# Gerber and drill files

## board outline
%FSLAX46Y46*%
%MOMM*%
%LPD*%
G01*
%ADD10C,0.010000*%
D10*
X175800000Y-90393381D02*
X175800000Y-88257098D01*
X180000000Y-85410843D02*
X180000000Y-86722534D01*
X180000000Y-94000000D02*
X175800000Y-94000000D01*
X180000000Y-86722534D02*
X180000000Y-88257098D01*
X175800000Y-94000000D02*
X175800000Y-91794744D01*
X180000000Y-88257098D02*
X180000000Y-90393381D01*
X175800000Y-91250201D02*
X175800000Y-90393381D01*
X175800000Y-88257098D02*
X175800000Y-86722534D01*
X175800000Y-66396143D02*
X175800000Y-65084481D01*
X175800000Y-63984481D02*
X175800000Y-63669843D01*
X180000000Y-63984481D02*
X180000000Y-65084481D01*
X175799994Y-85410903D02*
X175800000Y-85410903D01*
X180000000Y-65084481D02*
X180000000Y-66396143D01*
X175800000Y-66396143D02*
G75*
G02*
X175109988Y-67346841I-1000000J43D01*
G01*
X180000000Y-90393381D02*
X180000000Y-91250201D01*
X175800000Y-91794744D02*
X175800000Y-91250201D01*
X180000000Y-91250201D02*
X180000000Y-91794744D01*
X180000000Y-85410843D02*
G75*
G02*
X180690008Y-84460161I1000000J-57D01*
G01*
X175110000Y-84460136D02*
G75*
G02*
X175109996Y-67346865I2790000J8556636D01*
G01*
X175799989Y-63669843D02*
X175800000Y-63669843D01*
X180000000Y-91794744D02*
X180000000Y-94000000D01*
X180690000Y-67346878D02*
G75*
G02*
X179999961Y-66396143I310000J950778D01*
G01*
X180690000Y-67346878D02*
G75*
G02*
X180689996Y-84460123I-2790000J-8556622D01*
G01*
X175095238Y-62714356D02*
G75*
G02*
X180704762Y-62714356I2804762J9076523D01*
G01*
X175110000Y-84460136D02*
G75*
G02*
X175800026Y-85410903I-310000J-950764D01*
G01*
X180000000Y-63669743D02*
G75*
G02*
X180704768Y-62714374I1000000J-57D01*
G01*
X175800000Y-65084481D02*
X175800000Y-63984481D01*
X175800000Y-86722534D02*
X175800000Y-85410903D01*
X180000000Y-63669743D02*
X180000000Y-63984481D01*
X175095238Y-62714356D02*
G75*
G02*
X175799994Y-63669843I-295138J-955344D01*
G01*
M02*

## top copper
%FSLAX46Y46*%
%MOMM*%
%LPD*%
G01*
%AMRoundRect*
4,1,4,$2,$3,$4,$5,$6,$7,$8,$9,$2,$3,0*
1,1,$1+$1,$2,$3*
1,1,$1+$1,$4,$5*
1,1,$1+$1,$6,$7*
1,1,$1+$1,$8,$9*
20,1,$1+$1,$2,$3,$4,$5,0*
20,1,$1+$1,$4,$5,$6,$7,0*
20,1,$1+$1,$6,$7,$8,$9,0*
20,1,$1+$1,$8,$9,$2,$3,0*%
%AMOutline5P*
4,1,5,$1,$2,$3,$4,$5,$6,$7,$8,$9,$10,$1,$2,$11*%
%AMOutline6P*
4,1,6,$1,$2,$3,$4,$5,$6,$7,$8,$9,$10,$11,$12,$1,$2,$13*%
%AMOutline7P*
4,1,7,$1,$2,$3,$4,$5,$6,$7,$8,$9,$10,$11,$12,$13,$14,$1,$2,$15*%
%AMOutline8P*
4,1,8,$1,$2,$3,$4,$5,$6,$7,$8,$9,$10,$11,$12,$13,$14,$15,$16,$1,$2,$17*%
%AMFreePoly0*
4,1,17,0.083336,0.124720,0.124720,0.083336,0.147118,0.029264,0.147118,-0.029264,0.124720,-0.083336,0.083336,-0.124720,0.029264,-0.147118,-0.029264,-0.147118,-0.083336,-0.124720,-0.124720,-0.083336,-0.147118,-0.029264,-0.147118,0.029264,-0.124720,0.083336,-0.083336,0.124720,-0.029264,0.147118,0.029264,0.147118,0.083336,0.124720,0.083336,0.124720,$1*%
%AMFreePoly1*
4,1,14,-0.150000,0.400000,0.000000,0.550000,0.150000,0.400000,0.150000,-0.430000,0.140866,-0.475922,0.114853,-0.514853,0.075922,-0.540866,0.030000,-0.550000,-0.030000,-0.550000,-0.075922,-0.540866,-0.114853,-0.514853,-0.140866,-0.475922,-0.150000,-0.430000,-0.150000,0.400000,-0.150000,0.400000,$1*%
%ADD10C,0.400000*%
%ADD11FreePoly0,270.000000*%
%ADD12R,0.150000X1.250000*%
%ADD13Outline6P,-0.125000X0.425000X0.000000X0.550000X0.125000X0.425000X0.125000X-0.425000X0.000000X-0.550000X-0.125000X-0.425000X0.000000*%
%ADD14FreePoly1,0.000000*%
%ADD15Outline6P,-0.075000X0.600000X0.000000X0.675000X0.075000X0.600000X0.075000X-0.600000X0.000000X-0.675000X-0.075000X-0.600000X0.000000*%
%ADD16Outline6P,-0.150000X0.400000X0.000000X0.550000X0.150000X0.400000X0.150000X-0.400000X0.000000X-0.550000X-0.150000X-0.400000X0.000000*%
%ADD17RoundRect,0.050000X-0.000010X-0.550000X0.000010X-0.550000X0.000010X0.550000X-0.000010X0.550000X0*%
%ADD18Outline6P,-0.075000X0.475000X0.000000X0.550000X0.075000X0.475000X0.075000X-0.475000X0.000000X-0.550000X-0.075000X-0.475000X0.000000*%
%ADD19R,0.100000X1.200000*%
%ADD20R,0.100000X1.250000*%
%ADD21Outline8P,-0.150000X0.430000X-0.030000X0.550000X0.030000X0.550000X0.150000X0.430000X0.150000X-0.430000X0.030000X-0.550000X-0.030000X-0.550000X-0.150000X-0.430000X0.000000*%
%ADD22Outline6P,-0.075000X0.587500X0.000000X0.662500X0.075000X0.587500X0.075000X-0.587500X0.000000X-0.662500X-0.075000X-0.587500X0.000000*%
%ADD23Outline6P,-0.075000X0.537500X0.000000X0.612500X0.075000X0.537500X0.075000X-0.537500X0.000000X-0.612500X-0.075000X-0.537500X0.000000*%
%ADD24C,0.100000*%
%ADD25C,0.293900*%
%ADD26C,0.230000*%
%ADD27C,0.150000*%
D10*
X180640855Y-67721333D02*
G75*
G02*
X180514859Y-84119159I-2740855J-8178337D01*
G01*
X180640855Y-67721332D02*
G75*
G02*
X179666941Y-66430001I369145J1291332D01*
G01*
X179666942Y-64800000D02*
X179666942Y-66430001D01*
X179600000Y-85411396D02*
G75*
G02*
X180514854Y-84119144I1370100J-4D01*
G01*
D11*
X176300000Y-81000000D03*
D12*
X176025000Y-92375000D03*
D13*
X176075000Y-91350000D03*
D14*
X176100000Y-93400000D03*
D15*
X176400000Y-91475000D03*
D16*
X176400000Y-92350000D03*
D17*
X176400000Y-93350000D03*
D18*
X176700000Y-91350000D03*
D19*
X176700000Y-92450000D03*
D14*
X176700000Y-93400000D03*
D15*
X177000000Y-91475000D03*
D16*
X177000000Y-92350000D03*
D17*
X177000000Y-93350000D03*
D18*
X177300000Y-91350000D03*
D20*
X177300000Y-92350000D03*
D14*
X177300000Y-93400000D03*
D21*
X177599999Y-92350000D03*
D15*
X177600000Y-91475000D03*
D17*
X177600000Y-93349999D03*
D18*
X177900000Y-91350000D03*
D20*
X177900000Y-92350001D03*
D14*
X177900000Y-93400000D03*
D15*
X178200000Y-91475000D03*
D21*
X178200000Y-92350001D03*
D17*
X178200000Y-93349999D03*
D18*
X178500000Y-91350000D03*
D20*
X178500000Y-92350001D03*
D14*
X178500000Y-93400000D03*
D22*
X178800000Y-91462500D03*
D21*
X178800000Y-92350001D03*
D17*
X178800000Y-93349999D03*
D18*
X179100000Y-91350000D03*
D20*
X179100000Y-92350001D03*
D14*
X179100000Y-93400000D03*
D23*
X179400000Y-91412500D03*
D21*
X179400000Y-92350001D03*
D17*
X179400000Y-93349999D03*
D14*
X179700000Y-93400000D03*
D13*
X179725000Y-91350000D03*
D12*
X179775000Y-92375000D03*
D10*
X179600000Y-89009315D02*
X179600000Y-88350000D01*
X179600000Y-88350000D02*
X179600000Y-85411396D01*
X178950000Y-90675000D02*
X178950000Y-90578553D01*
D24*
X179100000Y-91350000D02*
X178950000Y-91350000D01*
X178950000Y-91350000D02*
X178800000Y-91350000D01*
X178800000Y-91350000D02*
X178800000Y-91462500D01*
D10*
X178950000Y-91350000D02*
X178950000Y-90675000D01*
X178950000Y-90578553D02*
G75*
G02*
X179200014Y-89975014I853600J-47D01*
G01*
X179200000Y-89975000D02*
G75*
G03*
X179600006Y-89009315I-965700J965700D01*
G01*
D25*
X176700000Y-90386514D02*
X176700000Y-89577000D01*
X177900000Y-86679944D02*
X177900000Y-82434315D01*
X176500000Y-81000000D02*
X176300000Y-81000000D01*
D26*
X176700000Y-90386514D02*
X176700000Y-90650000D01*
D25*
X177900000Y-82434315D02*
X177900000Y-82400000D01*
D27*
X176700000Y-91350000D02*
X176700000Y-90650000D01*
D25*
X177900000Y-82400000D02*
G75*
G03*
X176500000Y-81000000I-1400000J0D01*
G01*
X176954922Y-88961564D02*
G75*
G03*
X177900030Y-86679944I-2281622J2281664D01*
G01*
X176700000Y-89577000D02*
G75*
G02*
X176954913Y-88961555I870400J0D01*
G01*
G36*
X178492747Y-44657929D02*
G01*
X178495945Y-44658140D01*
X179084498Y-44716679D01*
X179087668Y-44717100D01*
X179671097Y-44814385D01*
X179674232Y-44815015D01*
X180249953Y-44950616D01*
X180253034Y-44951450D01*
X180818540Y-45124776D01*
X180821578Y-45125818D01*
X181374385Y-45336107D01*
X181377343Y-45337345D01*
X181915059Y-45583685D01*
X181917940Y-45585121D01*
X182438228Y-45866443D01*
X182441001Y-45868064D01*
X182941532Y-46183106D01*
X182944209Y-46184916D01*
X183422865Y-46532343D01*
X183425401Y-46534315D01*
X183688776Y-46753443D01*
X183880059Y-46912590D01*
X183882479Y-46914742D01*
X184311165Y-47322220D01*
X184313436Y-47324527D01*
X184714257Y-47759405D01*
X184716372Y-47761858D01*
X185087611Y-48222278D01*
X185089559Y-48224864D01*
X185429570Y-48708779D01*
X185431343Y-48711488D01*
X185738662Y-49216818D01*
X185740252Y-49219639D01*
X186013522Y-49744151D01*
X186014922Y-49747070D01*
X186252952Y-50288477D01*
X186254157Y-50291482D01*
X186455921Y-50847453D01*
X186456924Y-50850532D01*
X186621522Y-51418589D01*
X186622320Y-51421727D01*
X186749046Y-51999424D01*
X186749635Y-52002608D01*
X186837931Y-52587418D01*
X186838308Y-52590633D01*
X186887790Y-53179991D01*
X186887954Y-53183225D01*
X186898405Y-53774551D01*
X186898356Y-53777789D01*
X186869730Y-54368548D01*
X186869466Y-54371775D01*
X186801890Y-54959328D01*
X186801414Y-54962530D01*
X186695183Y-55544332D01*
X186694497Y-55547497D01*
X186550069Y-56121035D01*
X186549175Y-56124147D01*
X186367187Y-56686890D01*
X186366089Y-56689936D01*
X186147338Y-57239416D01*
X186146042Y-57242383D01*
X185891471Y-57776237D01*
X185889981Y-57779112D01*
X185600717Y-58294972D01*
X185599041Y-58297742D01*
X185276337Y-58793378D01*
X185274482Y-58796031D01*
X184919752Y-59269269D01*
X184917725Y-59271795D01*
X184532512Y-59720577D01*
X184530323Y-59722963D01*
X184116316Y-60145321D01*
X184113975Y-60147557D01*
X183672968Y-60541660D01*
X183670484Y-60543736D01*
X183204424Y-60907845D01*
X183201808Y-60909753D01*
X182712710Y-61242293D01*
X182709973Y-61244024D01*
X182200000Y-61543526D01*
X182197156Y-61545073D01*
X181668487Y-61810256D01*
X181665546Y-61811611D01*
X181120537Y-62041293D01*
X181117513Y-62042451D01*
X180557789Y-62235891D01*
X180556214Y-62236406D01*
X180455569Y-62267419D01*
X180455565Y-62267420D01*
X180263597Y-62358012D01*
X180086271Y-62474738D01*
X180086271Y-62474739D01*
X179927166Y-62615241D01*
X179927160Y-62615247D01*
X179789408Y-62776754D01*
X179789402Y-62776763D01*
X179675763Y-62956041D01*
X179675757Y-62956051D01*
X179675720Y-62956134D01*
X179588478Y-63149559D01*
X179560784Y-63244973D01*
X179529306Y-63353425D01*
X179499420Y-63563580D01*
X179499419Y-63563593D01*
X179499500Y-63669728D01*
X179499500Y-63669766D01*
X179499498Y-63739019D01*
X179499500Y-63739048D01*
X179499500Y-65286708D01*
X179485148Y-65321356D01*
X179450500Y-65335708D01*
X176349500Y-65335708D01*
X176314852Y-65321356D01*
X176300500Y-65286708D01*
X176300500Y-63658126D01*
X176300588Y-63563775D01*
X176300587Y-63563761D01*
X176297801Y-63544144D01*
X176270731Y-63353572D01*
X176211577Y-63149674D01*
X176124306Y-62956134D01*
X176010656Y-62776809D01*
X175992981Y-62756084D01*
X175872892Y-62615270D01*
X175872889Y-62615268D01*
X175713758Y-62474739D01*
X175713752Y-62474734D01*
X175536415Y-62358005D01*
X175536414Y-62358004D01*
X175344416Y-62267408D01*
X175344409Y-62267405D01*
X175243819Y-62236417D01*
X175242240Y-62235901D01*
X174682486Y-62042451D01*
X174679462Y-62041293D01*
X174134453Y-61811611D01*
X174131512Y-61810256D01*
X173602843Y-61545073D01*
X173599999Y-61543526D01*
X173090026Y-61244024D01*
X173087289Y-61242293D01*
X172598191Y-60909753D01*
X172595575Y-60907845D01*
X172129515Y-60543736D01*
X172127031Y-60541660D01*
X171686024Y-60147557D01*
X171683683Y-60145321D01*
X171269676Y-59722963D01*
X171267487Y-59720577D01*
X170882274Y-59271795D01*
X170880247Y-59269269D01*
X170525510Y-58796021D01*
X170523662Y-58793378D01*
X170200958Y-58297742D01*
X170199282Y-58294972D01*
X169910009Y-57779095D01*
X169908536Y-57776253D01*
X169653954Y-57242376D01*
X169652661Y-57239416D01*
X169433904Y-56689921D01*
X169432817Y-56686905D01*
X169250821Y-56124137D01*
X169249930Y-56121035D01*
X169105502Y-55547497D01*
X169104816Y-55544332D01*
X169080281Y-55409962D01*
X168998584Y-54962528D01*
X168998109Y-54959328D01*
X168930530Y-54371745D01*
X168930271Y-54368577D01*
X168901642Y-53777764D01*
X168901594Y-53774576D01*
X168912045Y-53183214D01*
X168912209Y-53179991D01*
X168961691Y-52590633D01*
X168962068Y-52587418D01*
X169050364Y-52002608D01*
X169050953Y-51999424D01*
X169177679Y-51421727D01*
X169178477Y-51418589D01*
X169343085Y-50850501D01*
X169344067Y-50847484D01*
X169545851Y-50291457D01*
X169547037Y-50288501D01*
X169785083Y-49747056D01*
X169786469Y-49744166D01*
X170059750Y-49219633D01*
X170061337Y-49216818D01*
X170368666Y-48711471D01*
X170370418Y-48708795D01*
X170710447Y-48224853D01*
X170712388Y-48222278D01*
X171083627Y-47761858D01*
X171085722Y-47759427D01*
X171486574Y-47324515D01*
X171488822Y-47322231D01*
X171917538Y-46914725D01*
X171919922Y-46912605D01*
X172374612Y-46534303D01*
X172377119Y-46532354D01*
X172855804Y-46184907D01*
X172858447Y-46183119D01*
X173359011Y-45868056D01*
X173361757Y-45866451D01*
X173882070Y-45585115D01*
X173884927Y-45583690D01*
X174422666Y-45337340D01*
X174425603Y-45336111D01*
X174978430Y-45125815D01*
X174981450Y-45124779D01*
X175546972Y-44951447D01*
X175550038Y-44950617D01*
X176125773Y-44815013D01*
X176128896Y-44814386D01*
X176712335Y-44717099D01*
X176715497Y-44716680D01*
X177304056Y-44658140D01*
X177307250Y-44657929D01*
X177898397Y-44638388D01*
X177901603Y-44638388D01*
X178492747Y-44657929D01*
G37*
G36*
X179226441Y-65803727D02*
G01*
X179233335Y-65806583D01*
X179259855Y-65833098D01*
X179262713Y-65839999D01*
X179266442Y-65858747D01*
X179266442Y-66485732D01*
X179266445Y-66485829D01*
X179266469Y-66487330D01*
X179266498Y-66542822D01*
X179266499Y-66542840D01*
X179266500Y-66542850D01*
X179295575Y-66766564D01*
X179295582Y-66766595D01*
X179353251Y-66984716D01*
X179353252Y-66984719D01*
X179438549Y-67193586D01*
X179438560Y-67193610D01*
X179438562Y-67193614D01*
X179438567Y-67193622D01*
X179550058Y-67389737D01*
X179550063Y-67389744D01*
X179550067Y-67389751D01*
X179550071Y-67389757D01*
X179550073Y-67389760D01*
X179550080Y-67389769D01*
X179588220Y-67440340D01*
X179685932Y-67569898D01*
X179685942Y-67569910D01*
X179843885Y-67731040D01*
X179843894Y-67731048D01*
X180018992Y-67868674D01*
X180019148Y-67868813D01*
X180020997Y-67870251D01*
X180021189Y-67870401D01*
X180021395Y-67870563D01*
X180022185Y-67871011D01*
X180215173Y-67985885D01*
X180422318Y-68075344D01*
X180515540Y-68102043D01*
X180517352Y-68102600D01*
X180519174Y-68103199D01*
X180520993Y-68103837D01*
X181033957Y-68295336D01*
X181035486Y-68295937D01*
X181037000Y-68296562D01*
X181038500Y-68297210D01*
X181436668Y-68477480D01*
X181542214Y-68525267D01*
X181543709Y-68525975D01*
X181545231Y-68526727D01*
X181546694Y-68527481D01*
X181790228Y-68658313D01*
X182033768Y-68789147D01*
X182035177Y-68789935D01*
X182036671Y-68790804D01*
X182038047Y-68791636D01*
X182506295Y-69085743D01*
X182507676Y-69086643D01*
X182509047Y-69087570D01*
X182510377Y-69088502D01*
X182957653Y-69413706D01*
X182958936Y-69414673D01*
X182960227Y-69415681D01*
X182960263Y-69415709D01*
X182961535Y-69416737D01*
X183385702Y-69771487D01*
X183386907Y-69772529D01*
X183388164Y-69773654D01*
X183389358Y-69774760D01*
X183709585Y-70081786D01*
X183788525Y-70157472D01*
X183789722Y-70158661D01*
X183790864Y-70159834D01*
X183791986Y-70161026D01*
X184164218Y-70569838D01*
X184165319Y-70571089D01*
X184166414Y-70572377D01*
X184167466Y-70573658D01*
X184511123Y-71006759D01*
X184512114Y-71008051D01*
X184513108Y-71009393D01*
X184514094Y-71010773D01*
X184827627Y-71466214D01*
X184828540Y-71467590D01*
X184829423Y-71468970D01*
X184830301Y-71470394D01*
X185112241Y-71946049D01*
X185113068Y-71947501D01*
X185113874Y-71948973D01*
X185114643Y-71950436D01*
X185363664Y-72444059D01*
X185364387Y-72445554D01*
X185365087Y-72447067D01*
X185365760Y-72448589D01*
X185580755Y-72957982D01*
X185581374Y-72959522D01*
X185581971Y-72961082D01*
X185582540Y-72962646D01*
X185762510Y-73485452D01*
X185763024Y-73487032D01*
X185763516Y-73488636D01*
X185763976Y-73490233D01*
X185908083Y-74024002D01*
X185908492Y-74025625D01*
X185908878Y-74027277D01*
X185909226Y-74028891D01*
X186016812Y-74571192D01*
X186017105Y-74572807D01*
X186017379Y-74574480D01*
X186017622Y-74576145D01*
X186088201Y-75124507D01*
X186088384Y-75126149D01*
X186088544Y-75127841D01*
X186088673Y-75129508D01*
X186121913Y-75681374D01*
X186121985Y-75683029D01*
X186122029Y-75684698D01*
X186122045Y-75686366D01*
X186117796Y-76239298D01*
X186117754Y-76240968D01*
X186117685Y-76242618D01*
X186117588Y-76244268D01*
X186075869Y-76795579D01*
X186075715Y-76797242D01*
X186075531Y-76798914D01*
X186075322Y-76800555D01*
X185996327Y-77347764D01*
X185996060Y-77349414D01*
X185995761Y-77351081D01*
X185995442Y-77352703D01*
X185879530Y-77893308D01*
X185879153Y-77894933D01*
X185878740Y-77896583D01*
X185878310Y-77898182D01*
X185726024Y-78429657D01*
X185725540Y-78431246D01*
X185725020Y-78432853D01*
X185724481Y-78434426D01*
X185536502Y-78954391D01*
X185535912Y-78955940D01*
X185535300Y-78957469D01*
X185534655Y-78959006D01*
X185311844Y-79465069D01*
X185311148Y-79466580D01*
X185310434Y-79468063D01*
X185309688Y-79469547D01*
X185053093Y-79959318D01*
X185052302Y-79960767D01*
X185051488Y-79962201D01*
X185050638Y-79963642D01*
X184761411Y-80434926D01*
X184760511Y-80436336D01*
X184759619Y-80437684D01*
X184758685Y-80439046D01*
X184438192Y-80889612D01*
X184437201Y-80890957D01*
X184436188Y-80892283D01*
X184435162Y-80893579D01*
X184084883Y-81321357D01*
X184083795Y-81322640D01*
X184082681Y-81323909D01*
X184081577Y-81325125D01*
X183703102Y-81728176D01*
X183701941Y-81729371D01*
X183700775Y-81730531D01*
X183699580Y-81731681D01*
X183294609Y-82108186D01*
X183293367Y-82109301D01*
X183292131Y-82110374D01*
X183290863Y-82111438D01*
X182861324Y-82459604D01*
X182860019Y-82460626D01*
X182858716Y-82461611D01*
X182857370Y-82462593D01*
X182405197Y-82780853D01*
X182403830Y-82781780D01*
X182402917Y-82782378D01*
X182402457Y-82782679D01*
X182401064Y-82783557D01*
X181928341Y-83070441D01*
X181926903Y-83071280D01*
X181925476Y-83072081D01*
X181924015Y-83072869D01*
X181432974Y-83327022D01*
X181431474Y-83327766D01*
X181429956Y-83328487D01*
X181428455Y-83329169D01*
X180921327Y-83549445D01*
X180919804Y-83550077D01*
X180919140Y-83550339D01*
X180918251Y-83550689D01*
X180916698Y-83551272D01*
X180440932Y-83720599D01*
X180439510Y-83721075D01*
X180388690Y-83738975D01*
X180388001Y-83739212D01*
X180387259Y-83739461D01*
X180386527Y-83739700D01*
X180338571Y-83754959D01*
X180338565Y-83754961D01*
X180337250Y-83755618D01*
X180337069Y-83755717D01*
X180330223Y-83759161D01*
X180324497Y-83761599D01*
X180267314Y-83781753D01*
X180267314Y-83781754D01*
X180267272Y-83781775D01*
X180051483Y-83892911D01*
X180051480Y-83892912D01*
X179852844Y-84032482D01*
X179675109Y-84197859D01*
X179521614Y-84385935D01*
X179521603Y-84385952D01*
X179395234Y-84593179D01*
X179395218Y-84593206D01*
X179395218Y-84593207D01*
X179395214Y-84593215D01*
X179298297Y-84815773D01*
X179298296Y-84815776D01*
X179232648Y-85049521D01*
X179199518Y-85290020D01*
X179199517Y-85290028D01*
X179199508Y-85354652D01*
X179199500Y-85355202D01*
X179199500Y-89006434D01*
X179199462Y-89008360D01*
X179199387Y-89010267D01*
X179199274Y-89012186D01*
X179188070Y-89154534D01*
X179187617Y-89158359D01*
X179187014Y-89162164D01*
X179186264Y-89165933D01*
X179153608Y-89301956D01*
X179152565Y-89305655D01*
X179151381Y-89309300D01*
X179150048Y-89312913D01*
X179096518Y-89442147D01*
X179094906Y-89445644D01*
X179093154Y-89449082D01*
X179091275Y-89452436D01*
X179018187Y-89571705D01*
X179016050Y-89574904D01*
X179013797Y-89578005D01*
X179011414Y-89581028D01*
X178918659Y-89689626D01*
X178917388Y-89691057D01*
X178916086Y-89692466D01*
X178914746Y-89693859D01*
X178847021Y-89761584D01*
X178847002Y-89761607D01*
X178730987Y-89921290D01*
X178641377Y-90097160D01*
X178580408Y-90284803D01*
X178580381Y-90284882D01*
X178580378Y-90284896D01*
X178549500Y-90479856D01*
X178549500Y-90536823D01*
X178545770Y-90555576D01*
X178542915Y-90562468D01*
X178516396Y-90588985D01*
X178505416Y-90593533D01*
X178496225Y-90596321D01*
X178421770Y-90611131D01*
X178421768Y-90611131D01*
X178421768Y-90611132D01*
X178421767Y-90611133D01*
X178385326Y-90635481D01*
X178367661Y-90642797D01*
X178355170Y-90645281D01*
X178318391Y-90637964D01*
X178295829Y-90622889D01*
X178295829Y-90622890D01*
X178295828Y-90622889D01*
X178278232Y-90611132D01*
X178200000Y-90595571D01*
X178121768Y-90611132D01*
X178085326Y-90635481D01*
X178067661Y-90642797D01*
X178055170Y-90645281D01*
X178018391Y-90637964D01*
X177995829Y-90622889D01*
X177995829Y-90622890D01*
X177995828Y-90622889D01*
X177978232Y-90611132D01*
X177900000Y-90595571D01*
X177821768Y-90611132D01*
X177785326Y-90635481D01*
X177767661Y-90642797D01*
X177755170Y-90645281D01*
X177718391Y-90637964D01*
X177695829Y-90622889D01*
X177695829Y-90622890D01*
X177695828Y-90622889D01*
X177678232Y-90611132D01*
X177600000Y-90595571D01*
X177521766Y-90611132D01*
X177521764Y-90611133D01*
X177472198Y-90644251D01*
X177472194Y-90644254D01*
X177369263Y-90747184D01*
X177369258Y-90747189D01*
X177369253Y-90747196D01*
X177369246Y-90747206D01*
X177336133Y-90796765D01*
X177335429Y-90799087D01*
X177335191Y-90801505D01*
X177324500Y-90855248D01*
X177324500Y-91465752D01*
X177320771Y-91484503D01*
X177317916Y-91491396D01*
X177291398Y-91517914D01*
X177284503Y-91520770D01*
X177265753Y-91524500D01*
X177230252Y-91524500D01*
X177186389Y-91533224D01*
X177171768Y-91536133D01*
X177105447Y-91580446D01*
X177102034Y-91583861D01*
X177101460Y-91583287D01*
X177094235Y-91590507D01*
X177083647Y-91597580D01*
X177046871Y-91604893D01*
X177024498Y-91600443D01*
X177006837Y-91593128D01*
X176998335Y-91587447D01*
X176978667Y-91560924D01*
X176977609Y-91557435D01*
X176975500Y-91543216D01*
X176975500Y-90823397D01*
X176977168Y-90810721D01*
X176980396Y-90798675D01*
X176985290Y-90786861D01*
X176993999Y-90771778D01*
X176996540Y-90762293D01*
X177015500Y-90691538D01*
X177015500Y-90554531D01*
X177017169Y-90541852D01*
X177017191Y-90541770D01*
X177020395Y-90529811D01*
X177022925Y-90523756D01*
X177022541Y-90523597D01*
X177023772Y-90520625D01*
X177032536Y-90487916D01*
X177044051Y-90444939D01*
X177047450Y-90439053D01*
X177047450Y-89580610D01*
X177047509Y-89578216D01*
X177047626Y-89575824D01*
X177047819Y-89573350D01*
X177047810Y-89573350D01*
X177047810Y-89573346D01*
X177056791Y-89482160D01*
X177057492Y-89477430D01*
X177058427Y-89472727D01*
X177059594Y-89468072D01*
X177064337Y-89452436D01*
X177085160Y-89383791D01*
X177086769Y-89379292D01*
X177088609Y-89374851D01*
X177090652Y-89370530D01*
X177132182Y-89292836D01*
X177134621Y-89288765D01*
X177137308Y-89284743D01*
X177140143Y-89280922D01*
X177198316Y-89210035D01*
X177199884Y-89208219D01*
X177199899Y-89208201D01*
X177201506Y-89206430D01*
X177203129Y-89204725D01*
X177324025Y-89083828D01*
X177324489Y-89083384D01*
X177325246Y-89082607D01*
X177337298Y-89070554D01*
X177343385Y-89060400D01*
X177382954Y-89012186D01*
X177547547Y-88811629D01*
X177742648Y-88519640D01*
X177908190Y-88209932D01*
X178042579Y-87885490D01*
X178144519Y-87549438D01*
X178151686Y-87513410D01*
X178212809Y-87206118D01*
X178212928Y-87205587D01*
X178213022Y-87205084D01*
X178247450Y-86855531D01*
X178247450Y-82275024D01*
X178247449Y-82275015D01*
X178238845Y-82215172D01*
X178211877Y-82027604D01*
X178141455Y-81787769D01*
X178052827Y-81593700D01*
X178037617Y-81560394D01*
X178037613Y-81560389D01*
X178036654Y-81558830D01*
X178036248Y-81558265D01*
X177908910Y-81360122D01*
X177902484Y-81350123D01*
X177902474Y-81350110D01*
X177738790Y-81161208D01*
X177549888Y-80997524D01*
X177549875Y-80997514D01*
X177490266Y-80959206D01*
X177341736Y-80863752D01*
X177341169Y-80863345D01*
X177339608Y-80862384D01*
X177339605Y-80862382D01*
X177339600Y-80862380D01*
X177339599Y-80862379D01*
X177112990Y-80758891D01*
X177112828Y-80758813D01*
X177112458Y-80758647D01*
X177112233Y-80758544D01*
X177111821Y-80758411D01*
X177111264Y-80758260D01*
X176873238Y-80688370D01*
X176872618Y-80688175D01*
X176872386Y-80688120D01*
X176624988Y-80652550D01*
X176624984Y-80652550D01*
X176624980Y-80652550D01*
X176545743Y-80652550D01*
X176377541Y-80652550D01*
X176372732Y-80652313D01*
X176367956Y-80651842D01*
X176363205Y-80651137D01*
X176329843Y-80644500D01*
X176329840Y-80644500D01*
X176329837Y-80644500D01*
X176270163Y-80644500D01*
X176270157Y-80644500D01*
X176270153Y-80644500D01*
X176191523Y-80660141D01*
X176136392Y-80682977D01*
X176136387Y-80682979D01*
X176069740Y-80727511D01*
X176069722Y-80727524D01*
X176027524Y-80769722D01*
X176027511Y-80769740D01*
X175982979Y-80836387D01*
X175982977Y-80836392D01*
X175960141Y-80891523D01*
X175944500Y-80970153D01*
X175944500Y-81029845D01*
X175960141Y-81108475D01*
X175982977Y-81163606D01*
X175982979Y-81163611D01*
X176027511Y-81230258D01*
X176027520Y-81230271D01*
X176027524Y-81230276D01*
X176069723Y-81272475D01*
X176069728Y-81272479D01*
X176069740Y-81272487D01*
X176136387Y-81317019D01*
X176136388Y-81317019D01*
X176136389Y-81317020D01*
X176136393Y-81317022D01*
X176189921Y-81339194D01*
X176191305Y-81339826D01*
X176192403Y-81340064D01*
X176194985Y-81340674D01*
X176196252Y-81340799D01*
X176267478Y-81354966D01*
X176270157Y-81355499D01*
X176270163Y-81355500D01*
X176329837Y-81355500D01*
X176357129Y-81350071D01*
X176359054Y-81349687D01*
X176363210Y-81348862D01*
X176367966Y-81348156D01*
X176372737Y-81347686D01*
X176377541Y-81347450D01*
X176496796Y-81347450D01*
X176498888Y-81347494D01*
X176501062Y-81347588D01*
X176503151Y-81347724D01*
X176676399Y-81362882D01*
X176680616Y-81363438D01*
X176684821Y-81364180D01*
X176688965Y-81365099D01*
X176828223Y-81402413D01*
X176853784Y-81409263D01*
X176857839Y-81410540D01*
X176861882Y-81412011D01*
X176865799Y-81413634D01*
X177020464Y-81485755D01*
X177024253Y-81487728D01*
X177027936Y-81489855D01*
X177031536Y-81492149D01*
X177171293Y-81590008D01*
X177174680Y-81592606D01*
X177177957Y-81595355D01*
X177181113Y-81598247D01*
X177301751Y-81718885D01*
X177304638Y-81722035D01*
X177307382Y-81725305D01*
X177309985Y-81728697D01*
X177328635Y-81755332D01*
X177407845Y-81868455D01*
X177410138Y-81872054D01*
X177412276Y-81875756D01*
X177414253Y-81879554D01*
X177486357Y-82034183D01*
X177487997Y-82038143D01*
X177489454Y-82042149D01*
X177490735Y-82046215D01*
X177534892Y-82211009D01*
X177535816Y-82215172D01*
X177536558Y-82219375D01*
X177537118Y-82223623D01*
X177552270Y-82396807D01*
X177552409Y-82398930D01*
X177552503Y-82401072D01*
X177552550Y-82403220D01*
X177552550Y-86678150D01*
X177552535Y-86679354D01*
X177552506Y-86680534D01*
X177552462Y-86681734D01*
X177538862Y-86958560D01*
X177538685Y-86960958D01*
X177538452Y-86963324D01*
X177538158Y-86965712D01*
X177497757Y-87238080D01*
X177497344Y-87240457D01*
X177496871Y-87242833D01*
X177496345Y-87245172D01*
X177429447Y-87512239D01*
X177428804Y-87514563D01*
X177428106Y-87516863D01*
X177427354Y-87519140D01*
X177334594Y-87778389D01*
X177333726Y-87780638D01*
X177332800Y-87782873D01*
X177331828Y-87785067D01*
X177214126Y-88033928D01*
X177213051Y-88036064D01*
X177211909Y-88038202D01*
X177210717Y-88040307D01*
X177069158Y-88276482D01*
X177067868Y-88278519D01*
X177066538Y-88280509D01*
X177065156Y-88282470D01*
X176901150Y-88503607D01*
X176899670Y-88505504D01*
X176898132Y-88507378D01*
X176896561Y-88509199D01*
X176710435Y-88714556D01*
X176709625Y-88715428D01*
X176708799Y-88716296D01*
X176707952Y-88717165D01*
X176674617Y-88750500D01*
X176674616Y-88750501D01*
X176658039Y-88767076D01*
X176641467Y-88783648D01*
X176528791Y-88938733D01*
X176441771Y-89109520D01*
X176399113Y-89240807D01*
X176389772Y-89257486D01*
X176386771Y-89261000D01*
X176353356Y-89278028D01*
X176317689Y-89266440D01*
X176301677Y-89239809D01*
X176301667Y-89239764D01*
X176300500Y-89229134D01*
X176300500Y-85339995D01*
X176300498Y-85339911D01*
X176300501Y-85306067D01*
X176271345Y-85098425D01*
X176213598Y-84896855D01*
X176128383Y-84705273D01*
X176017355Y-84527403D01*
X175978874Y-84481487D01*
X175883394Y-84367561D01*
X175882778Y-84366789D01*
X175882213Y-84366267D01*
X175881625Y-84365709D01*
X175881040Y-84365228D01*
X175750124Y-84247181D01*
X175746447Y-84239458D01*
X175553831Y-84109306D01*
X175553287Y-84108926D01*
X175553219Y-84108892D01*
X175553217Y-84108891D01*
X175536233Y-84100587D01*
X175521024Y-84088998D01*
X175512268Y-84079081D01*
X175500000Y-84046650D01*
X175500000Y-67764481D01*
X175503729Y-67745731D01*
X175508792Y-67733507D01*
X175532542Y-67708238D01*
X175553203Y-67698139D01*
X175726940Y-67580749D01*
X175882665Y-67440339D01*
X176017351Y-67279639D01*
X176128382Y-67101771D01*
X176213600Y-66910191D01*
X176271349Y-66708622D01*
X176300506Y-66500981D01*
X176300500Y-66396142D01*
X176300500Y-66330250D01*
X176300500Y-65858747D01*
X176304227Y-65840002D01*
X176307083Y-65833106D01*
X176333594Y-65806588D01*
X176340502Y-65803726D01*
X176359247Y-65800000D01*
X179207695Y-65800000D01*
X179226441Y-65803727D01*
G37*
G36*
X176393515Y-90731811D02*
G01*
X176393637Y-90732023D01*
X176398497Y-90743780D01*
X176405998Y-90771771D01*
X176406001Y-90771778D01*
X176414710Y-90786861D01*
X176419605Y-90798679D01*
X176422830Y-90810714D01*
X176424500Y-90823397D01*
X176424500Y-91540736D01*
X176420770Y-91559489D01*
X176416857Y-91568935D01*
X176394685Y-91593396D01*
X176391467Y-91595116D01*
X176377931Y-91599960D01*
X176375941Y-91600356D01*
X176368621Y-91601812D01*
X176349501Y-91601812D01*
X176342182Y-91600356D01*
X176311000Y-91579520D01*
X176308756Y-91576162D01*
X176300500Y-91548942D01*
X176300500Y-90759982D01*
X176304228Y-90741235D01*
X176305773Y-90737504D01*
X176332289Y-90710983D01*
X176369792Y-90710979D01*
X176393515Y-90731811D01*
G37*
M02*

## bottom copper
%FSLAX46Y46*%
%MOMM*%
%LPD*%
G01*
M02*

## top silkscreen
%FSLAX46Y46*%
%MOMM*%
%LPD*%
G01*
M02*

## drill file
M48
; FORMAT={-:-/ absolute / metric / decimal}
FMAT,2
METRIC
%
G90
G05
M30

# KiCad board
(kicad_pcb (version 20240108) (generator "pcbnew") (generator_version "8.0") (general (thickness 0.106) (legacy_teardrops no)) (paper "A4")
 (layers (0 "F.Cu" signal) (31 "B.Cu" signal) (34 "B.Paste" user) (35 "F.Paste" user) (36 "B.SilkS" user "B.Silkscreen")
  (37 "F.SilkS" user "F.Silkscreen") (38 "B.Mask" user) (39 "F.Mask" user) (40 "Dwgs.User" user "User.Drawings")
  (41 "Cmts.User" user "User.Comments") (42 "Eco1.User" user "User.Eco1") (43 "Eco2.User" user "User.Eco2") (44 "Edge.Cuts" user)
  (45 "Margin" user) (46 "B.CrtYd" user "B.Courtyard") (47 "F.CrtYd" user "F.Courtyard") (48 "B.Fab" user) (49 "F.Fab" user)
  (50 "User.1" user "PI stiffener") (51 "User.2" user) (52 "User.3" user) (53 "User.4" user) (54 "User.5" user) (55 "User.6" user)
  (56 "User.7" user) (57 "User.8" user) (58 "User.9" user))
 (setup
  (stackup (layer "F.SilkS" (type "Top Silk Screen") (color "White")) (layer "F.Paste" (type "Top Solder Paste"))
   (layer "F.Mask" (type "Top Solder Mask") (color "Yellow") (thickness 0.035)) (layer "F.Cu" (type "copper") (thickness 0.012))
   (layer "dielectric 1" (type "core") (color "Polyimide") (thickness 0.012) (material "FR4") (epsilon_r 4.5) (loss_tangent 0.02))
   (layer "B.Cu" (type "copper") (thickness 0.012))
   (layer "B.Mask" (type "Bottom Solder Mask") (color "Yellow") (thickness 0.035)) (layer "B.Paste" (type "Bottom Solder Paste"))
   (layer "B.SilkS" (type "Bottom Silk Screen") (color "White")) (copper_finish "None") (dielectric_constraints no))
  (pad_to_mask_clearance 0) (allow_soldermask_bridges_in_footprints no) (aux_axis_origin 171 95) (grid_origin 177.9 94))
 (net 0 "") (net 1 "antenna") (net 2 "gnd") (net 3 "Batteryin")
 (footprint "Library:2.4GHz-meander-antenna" (layer "F.Cu") (at 176.3 81 -90)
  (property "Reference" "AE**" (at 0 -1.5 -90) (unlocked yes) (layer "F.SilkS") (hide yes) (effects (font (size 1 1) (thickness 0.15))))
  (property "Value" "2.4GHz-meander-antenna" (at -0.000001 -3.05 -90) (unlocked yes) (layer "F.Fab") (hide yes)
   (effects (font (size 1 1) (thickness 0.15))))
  (pad "1" smd custom (at 0 0 270) (size 0.3 0.3) (layers "F.Cu") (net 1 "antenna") (thermal_bridge_angle 90)
   (options (clearance outline) (anchor circle)) (primitives)))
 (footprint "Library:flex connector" (layer "B.Cu") (at 175.7 90.05)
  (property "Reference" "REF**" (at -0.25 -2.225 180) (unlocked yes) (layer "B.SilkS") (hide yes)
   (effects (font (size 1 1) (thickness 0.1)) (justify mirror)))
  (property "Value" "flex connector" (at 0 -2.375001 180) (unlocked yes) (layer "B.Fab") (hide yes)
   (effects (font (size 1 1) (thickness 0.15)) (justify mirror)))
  (pad "1" smd rect (at 0.325 2.325) (size 0.15 1.25) (layers "F.Cu" "F.Paste" "F.Mask") (thermal_bridge_angle 45))
  (pad "1" smd roundrect (at 0.375 1.3) (size 0.25 1.1) (layers "F.Cu" "F.Paste" "F.Mask") (roundrect_rratio 0) (chamfer_ratio 0.5)
   (chamfer top_left top_right bottom_left bottom_right) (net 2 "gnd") (thermal_bridge_angle 45))
  (pad "1" smd roundrect (at 0.4 3.35) (size 0.3 1.1) (layers "F.Cu" "F.Paste" "F.Mask") (roundrect_rratio 0.4) (chamfer_ratio 0.5)
   (chamfer top_left top_right) (thermal_bridge_angle 45))
  (pad "2" smd roundrect (at 0.7 1.425) (size 0.15 1.35) (layers "F.Cu" "F.Paste" "F.Mask") (roundrect_rratio 0) (chamfer_ratio 0.5)
   (chamfer top_left top_right bottom_left bottom_right) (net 2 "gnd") (thermal_bridge_angle 45))
  (pad "2" smd roundrect (at 0.7 2.3) (size 0.3 1.1) (layers "F.Cu" "F.Paste" "F.Mask") (roundrect_rratio 0) (chamfer_ratio 0.5)
   (chamfer top_left top_right bottom_left bottom_right) (thermal_bridge_angle 45))
  (pad "2" smd roundrect (at 0.7 3.3) (size 0.1 1.2) (layers "F.Cu" "F.Paste" "F.Mask") (roundrect_rratio 0.5) (thermal_bridge_angle 45))
  (pad "3" smd roundrect (at 1 1.3) (size 0.15 1.1) (layers "F.Cu" "F.Paste" "F.Mask") (roundrect_rratio 0) (chamfer_ratio 0.5)
   (chamfer top_left top_right bottom_left bottom_right) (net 1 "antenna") (thermal_bridge_angle 45))
  (pad "3" smd rect (at 1 2.4) (size 0.1 1.2) (layers "F.Cu" "F.Paste" "F.Mask") (thermal_bridge_angle 45))
  (pad "3" smd roundrect (at 1 3.35) (size 0.3 1.1) (layers "F.Cu" "F.Paste" "F.Mask") (roundrect_rratio 0.4) (chamfer_ratio 0.5)
   (chamfer top_left top_right) (thermal_bridge_angle 45))
  (pad "4" smd roundrect (at 1.3 1.425) (size 0.15 1.35) (layers "F.Cu" "F.Paste" "F.Mask") (roundrect_rratio 0) (chamfer_ratio 0.5)
   (chamfer top_left top_right bottom_left bottom_right) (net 2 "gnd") (thermal_bridge_angle 45))
  (pad "4" smd roundrect (at 1.3 2.3) (size 0.3 1.1) (layers "F.Cu" "F.Paste" "F.Mask") (roundrect_rratio 0) (chamfer_ratio 0.5)
   (chamfer top_left top_right bottom_left bottom_right) (thermal_bridge_angle 45))
  (pad "4" smd roundrect (at 1.3 3.3) (size 0.1 1.2) (layers "F.Cu" "F.Paste" "F.Mask") (roundrect_rratio 0.5) (thermal_bridge_angle 45))
  (pad "5" smd roundrect (at 1.6 1.3) (size 0.15 1.1) (layers "F.Cu" "F.Paste" "F.Mask") (roundrect_rratio 0) (chamfer_ratio 0.5)
   (chamfer top_left top_right bottom_left bottom_right) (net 2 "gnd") (thermal_bridge_angle 45))
  (pad "5" smd rect (at 1.6 2.3) (size 0.1 1.25) (layers "F.Cu" "F.Paste" "F.Mask") (thermal_bridge_angle 45))
  (pad "5" smd roundrect (at 1.6 3.35) (size 0.3 1.1) (layers "F.Cu" "F.Paste" "F.Mask") (roundrect_rratio 0.4) (chamfer_ratio 0.5)
   (chamfer top_left top_right) (thermal_bridge_angle 45))
  (pad "6" smd roundrect (at 1.899999 2.3) (size 0.3 1.1) (layers "F.Cu" "F.Paste" "F.Mask") (roundrect_rratio 0) (chamfer_ratio 0.4)
   (chamfer top_left top_right bottom_left bottom_right) (thermal_bridge_angle 45))
  (pad "6" smd roundrect (at 1.9 1.425) (size 0.15 1.35) (layers "F.Cu" "F.Paste" "F.Mask") (roundrect_rratio 0) (chamfer_ratio 0.5)
   (chamfer top_left top_right bottom_left bottom_right) (thermal_bridge_angle 45))
  (pad "6" smd roundrect (at 1.9 3.299999) (size 0.1 1.2) (layers "F.Cu" "F.Paste" "F.Mask") (roundrect_rratio 0.5)
   (thermal_bridge_angle 45))
  (pad "7" smd roundrect (at 2.2 1.3) (size 0.15 1.1) (layers "F.Cu" "F.Paste" "F.Mask") (roundrect_rratio 0) (chamfer_ratio 0.5)
   (chamfer top_left top_right bottom_left bottom_right) (thermal_bridge_angle 45))
  (pad "7" smd rect (at 2.2 2.300001) (size 0.1 1.25) (layers "F.Cu" "F.Paste" "F.Mask") (thermal_bridge_angle 45))
  (pad "7" smd roundrect (at 2.2 3.35) (size 0.3 1.1) (layers "F.Cu" "F.Paste" "F.Mask") (roundrect_rratio 0.4) (chamfer_ratio 0.5)
   (chamfer top_left top_right) (thermal_bridge_angle 45))
  (pad "8" smd roundrect (at 2.5 1.425) (size 0.15 1.35) (layers "F.Cu" "F.Paste" "F.Mask") (roundrect_rratio 0) (chamfer_ratio 0.5)
   (chamfer top_left top_right bottom_left bottom_right) (thermal_bridge_angle 45))
  (pad "8" smd roundrect (at 2.5 2.300001) (size 0.3 1.1) (layers "F.Cu" "F.Paste" "F.Mask") (roundrect_rratio 0) (chamfer_ratio 0.4)
   (chamfer top_left top_right bottom_left bottom_right) (thermal_bridge_angle 45))
  (pad "8" smd roundrect (at 2.5 3.299999) (size 0.1 1.2) (layers "F.Cu" "F.Paste" "F.Mask") (roundrect_rratio 0.5)
   (thermal_bridge_angle 45))
  (pad "9" smd roundrect (at 2.8 1.3) (size 0.15 1.1) (layers "F.Cu" "F.Paste" "F.Mask") (roundrect_rratio 0) (chamfer_ratio 0.5)
   (chamfer top_left top_right bottom_left bottom_right) (thermal_bridge_angle 45))
  (pad "9" smd rect (at 2.8 2.300001) (size 0.1 1.25) (layers "F.Cu" "F.Paste" "F.Mask") (thermal_bridge_angle 45))
  (pad "9" smd roundrect (at 2.8 3.35) (size 0.3 1.1) (layers "F.Cu" "F.Paste" "F.Mask") (roundrect_rratio 0.4) (chamfer_ratio 0.5)
   (chamfer top_left top_right) (thermal_bridge_angle 45))
  (pad "10" smd roundrect (at 3.1 1.4125) (size 0.15 1.325) (layers "F.Cu" "F.Paste" "F.Mask") (roundrect_rratio 0) (chamfer_ratio 0.5)
   (chamfer top_left top_right bottom_left bottom_right) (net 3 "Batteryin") (thermal_bridge_angle 45))
  (pad "10" smd roundrect (at 3.1 2.300001) (size 0.3 1.1) (layers "F.Cu" "F.Paste" "F.Mask") (roundrect_rratio 0) (chamfer_ratio 0.4)
   (chamfer top_left top_right bottom_left bottom_right) (thermal_bridge_angle 45))
  (pad "10" smd roundrect (at 3.1 3.299999) (size 0.1 1.2) (layers "F.Cu" "F.Paste" "F.Mask") (roundrect_rratio 0.5)
   (thermal_bridge_angle 45))
  (pad "11" smd roundrect (at 3.4 1.3) (size 0.15 1.1) (layers "F.Cu" "F.Paste" "F.Mask") (roundrect_rratio 0) (chamfer_ratio 0.5)
   (chamfer top_left top_right bottom_left bottom_right) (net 3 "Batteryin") (thermal_bridge_angle 45))
  (pad "11" smd rect (at 3.4 2.300001) (size 0.1 1.25) (layers "F.Cu" "F.Paste" "F.Mask") (thermal_bridge_angle 45))
  (pad "11" smd roundrect (at 3.4 3.35) (size 0.3 1.1) (layers "F.Cu" "F.Paste" "F.Mask") (roundrect_rratio 0.4) (chamfer_ratio 0.5)
   (chamfer top_left top_right) (thermal_bridge_angle 45))
  (pad "12" smd roundrect (at 3.7 1.3625) (size 0.15 1.225) (layers "F.Cu" "F.Paste" "F.Mask") (roundrect_rratio 0) (chamfer_ratio 0.5)
   (chamfer top_left top_right bottom_left bottom_right) (thermal_bridge_angle 45))
  (pad "12" smd roundrect (at 3.7 2.300001) (size 0.3 1.1) (layers "F.Cu" "F.Paste" "F.Mask") (roundrect_rratio 0) (chamfer_ratio 0.4)
   (chamfer top_left top_right bottom_left bottom_right) (thermal_bridge_angle 45))
  (pad "12" smd roundrect (at 3.7 3.299999) (size 0.1 1.2) (layers "F.Cu" "F.Paste" "F.Mask") (roundrect_rratio 0.5)
   (thermal_bridge_angle 45))
  (pad "13" smd roundrect (at 4 3.35) (size 0.3 1.1) (layers "F.Cu" "F.Paste" "F.Mask") (roundrect_rratio 0.4) (chamfer_ratio 0.5)
   (chamfer top_left top_right) (thermal_bridge_angle 45))
  (pad "13" smd roundrect (at 4.025 1.3) (size 0.25 1.1) (layers "F.Cu" "F.Paste" "F.Mask") (roundrect_rratio 0) (chamfer_ratio 0.5)
   (chamfer top_left top_right bottom_left bottom_right) (thermal_bridge_angle 45))
  (pad "13" smd rect (at 4.075 2.325) (size 0.15 1.25) (layers "F.Cu" "F.Paste" "F.Mask") (thermal_bridge_angle 45)))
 (gr_arc (start 180.640855 67.721333) (mid 186.525141 75.965942) (end 180.514858 84.119155) (stroke (width 0.4) (type default))
  (layer "F.Cu") (net 3))
 (gr_arc (start 180.640855 67.721332) (mid 179.937716 67.23871) (end 179.666942 66.430001) (stroke (width 0.4) (type default))
  (layer "F.Cu") (net 3))
 (gr_line (start 179.666942 64.8) (end 179.666942 66.430001) (stroke (width 0.4) (type default)) (layer "F.Cu") (net 3))
 (gr_arc (start 179.6 85.411396) (mid 179.851865 84.619744) (end 180.514858 84.119156) (stroke (width 0.4) (type default)) (layer "F.Cu")
  (net 3))
 (gr_line (start 175.8 90.393381) (end 175.8 88.257098) (stroke (width 0.01) (type default)) (layer "Edge.Cuts"))
 (gr_line (start 180 85.410843) (end 180 86.722534) (stroke (width 0.01) (type default)) (layer "Edge.Cuts"))
 (gr_line (start 180 94) (end 175.8 94) (stroke (width 0.01) (type default)) (layer "Edge.Cuts"))
 (gr_line (start 180 86.722534) (end 180 88.257098) (stroke (width 0.01) (type default)) (layer "Edge.Cuts"))
 (gr_line (start 175.8 94) (end 175.8 91.794744) (stroke (width 0.01) (type default)) (layer "Edge.Cuts"))
 (gr_line (start 180 88.257098) (end 180 90.393381) (stroke (width 0.01) (type default)) (layer "Edge.Cuts"))
 (gr_line (start 175.8 91.250201) (end 175.8 90.393381) (stroke (width 0.01) (type default)) (layer "Edge.Cuts"))
 (gr_line (start 175.8 88.257098) (end 175.8 86.722534) (stroke (width 0.01) (type default)) (layer "Edge.Cuts"))
 (gr_line (start 175.8 66.396143) (end 175.8 65.084481) (stroke (width 0.01) (type default)) (layer "Edge.Cuts"))
 (gr_line (start 175.8 63.984481) (end 175.8 63.669843) (stroke (width 0.01) (type default)) (layer "Edge.Cuts"))
 (gr_line (start 180 63.984481) (end 180 65.084481) (stroke (width 0.01) (type default)) (layer "Edge.Cuts"))
 (gr_line (start 175.799994 85.410903) (end 175.8 85.410903) (stroke (width 0.01) (type default)) (layer "Edge.Cuts"))
 (gr_line (start 180 65.084481) (end 180 66.396143) (stroke (width 0.01) (type default)) (layer "Edge.Cuts"))
 (gr_arc (start 175.8 66.396143) (mid 175.609321 66.98351) (end 175.11 67.346878) (stroke (width 0.01) (type default)) (layer "Edge.Cuts"))
 (gr_line (start 180 90.393381) (end 180 91.250201) (stroke (width 0.01) (type default)) (layer "Edge.Cuts"))
 (gr_line (start 175.8 91.794744) (end 175.8 91.250201) (stroke (width 0.01) (type default)) (layer "Edge.Cuts"))
 (gr_line (start 180 91.250201) (end 180 91.794744) (stroke (width 0.01) (type default)) (layer "Edge.Cuts"))
 (gr_arc (start 180 85.410843) (mid 180.190685 84.8235) (end 180.69 84.460136) (stroke (width 0.01) (type default)) (layer "Edge.Cuts"))
 (gr_arc (start 175.11 84.460136) (mid 168.9 75.903507) (end 175.11 67.346878) (stroke (width 0.01) (type default)) (layer "Edge.Cuts"))
 (gr_line (start 175.799989 63.669843) (end 175.8 63.669843) (stroke (width 0.01) (type default)) (layer "Edge.Cuts"))
 (gr_line (start 180 91.794744) (end 180 94) (stroke (width 0.01) (type default)) (layer "Edge.Cuts"))
 (gr_arc (start 180.69 67.346878) (mid 180.19068 66.983509) (end 180 66.396143) (stroke (width 0.01) (type default)) (layer "Edge.Cuts"))
 (gr_arc (start 180.69 67.346878) (mid 186.9 75.903507) (end 180.69 84.460136) (stroke (width 0.01) (type default)) (layer "Edge.Cuts"))
 (gr_arc (start 175.095238 62.714356) (mid 177.9 44.137835) (end 180.704762 62.714356) (stroke (width 0.01) (type default))
  (layer "Edge.Cuts"))
 (gr_arc (start 175.11 84.460136) (mid 175.609319 84.823524) (end 175.799994 85.410903) (stroke (width 0.01) (type default))
  (layer "Edge.Cuts"))
 (gr_arc (start 180 63.669743) (mid 180.195258 63.076151) (end 180.704762 62.714356) (stroke (width 0.01) (type default))
  (layer "Edge.Cuts"))
 (gr_line (start 175.8 65.084481) (end 175.8 63.984481) (stroke (width 0.01) (type default)) (layer "Edge.Cuts"))
 (gr_line (start 175.8 86.722534) (end 175.8 85.410903) (stroke (width 0.01) (type default)) (layer "Edge.Cuts"))
 (gr_line (start 180 63.669743) (end 180 63.984481) (stroke (width 0.01) (type default)) (layer "Edge.Cuts"))
 (gr_arc (start 175.095238 62.714356) (mid 175.604791 63.076183) (end 175.799989 63.669843) (stroke (width 0.01) (type default))
  (layer "Edge.Cuts"))
 (segment (start 179.6 89.009315) (end 179.6 88.35) (width 0.4) (layer "F.Cu") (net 3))
 (segment (start 179.6 88.35) (end 179.6 85.411396) (width 0.4) (layer "F.Cu") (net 3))
 (segment (start 178.95 90.675) (end 178.95 90.578553) (width 0.4) (layer "F.Cu") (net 3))
 (segment (start 179.1 91.35) (end 178.95 91.35) (width 0.1) (layer "F.Cu") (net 3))
 (segment (start 178.95 91.35) (end 178.8 91.35) (width 0.1) (layer "F.Cu") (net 3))
 (segment (start 178.8 91.35) (end 178.8 91.4625) (width 0.1) (layer "F.Cu") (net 3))
 (segment (start 178.95 91.35) (end 178.95 90.675) (width 0.4) (layer "F.Cu") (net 3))
 (arc (start 178.95 90.578553) (mid 179.014973 90.251913) (end 179.2 89.975) (width 0.4) (layer "F.Cu") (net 3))
 (arc (start 179.2 89.975) (mid 179.496044 89.53194) (end 179.6 89.009315) (width 0.4) (layer "F.Cu") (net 3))
 (segment (start 176.7 90.386514) (end 176.7 89.577) (width 0.2939) (layer "F.Cu") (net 1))
 (segment (start 177.9 86.679944) (end 177.9 82.434315) (width 0.2939) (layer "F.Cu") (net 1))
 (segment (start 176.5 81) (end 176.3 81) (width 0.2939) (layer "F.Cu") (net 1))
 (segment (start 176.7 90.386514) (end 176.7 90.65) (width 0.23) (layer "F.Cu") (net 1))
 (segment (start 177.9 82.434315) (end 177.9 82.4) (width 0.2939) (layer "F.Cu") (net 1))
 (segment (start 176.7 91.35) (end 176.7 90.65) (width 0.15) (layer "F.Cu") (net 1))
 (arc (start 177.9 82.4) (mid 177.489949 81.410051) (end 176.5 81) (width 0.2939) (layer "F.Cu") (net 1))
 (arc (start 176.954922 88.961564) (mid 177.654383 87.914748) (end 177.9 86.679944) (width 0.2939) (layer "F.Cu") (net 1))
 (arc (start 176.7 89.577) (mid 176.766252 89.243929) (end 176.954922 88.961564) (width 0.2939) (layer "F.Cu") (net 1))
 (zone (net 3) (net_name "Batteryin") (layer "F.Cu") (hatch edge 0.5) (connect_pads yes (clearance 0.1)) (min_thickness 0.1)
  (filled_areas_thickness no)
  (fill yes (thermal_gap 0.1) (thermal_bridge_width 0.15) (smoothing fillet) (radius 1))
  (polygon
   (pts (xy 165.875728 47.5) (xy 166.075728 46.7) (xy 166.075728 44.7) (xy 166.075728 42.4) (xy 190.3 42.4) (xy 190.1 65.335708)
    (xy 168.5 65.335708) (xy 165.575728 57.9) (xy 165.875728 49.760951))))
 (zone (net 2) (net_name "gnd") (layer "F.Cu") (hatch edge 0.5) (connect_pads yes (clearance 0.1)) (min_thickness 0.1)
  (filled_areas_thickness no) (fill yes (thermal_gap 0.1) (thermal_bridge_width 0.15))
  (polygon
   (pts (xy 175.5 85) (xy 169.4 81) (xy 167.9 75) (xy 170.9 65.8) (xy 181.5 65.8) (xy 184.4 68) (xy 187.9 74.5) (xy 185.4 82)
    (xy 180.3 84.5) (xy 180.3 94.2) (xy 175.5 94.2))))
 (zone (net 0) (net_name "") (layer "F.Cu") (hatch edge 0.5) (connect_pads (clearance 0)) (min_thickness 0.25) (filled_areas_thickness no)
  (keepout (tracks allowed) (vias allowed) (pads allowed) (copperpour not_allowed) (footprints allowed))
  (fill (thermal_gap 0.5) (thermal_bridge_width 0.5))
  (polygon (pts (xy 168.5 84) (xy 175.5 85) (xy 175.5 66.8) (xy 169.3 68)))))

